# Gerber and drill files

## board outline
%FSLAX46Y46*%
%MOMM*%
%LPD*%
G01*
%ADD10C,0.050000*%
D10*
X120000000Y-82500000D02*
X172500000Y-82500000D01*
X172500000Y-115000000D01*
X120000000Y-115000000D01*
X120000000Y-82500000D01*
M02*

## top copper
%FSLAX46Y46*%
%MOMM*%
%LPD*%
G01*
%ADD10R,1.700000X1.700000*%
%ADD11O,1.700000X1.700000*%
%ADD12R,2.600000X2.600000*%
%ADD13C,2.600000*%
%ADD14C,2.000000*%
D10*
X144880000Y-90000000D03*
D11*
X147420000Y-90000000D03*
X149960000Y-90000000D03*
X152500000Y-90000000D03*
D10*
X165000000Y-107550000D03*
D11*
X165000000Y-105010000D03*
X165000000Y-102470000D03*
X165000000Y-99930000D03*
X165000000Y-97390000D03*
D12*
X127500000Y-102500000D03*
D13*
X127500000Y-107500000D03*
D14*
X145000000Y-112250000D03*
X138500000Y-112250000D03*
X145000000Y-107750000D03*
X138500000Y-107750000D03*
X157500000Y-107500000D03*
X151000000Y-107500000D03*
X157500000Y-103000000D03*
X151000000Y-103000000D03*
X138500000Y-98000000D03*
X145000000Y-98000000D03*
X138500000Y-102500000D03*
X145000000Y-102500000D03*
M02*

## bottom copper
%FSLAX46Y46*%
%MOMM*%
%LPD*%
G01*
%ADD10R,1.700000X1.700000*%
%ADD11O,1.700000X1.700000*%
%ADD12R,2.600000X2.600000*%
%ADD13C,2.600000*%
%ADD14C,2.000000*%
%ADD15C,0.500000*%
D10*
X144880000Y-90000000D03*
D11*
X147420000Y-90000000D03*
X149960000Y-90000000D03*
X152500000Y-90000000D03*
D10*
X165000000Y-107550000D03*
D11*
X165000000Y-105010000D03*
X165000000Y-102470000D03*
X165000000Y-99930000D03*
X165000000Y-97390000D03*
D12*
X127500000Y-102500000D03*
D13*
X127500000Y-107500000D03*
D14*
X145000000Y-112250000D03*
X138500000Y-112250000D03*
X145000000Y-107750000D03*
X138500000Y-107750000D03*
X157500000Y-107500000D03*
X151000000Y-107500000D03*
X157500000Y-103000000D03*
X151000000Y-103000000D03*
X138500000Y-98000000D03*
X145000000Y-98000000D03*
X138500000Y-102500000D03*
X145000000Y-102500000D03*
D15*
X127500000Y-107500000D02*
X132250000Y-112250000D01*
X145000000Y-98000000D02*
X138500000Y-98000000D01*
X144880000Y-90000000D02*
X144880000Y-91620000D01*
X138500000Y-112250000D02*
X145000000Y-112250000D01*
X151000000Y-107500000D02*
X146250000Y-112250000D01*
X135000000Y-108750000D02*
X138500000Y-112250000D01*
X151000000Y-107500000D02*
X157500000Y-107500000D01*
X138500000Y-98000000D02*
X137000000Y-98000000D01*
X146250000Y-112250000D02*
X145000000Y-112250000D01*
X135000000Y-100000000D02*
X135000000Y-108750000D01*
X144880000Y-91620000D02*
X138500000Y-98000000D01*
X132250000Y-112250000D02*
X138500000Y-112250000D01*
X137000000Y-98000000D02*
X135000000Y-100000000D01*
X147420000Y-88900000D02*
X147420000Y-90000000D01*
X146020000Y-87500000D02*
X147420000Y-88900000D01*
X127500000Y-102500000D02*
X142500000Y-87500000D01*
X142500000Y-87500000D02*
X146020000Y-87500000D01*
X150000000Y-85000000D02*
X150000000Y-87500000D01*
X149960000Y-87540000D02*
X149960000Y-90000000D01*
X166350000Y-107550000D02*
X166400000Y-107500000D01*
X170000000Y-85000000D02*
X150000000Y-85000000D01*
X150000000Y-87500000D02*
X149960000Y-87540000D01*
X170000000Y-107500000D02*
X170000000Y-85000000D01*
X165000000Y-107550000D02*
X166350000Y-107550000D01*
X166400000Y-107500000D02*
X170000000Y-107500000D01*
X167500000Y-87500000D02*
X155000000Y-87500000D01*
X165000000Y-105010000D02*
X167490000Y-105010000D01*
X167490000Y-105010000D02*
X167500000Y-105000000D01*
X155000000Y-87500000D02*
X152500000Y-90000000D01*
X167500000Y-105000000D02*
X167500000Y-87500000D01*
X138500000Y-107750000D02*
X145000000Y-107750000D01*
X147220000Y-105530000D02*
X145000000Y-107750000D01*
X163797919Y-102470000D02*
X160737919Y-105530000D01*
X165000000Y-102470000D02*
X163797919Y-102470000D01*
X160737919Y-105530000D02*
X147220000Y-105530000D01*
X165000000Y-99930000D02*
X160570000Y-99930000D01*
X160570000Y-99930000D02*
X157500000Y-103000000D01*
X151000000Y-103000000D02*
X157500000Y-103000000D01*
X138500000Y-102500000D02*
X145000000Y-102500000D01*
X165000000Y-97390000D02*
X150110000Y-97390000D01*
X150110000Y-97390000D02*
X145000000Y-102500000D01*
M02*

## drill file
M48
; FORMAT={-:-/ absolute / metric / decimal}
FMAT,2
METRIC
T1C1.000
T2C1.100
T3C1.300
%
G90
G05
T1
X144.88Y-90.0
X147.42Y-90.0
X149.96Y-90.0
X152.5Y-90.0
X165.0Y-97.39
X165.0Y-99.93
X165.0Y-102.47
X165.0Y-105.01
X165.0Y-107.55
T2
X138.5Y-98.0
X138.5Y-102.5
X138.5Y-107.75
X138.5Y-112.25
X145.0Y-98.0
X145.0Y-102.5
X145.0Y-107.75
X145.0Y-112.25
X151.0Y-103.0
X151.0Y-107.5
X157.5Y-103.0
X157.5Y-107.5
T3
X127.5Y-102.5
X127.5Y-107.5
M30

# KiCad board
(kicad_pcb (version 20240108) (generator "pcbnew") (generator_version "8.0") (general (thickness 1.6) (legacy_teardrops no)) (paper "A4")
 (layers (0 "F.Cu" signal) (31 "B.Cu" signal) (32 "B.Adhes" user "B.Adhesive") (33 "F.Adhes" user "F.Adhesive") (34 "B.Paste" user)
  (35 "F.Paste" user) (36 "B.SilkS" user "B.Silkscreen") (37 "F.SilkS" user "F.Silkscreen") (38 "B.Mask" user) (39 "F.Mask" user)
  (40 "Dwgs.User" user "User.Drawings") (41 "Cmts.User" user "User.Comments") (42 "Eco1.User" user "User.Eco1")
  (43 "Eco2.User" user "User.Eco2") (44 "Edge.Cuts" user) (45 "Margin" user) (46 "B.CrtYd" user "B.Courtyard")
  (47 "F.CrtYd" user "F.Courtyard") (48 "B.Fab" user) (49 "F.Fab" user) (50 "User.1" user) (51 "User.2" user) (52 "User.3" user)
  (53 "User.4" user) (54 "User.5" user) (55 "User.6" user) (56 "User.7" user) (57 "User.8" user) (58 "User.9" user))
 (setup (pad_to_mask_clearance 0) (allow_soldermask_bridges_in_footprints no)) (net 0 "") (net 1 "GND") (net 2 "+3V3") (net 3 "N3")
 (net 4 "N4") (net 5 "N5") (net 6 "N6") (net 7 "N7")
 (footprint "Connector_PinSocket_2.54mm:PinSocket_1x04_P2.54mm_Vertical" (layer "F.Cu") (at 144.88 90 90)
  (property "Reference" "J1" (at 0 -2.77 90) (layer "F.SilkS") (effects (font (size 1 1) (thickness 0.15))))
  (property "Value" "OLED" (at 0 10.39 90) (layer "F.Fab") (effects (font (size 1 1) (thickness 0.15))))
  (pad "1" thru_hole rect (at 0 0 90) (size 1.7 1.7) (drill 1) (layers "*.Cu" "*.Mask") (remove_unused_layers no) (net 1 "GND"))
  (pad "2" thru_hole oval (at 0 2.54 90) (size 1.7 1.7) (drill 1) (layers "*.Cu" "*.Mask") (remove_unused_layers no) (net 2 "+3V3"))
  (pad "3" thru_hole oval (at 0 5.08 90) (size 1.7 1.7) (drill 1) (layers "*.Cu" "*.Mask") (remove_unused_layers no) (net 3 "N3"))
  (pad "4" thru_hole oval (at 0 7.62 90) (size 1.7 1.7) (drill 1) (layers "*.Cu" "*.Mask") (remove_unused_layers no) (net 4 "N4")))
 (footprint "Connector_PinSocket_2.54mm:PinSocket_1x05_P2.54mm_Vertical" (layer "F.Cu") (at 165 107.55 180)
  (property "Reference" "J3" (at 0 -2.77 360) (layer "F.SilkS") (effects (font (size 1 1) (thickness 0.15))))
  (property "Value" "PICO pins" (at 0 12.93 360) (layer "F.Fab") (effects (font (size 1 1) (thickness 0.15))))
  (pad "1" thru_hole rect (at 0 0 180) (size 1.7 1.7) (drill 1) (layers "*.Cu" "*.Mask") (remove_unused_layers no) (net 3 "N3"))
  (pad "2" thru_hole oval (at 0 2.54 180) (size 1.7 1.7) (drill 1) (layers "*.Cu" "*.Mask") (remove_unused_layers no) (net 4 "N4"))
  (pad "3" thru_hole oval (at 0 5.08 180) (size 1.7 1.7) (drill 1) (layers "*.Cu" "*.Mask") (remove_unused_layers no) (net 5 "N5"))
  (pad "4" thru_hole oval (at 0 7.62 180) (size 1.7 1.7) (drill 1) (layers "*.Cu" "*.Mask") (remove_unused_layers no) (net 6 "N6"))
  (pad "5" thru_hole oval (at 0 10.16 180) (size 1.7 1.7) (drill 1) (layers "*.Cu" "*.Mask") (remove_unused_layers no) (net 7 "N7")))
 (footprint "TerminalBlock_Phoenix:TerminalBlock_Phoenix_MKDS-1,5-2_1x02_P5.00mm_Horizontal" (layer "F.Cu") (at 127.5 102.5 -90)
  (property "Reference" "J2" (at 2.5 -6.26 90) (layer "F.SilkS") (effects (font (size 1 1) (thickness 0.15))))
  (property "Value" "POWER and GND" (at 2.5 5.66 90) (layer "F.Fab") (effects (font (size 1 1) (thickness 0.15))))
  (pad "1" thru_hole rect (at 0 0 270) (size 2.6 2.6) (drill 1.3) (layers "*.Cu" "*.Mask") (remove_unused_layers no) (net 2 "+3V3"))
  (pad "2" thru_hole circle (at 5 0 270) (size 2.6 2.6) (drill 1.3) (layers "*.Cu" "*.Mask") (remove_unused_layers no) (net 1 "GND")))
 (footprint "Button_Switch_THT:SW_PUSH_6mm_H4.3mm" (layer "F.Cu") (at 145 112.25 180)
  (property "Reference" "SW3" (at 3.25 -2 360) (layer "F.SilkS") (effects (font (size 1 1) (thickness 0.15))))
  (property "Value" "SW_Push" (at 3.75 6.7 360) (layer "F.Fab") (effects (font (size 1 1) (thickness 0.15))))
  (pad "1" thru_hole circle (at 0 0 270) (size 2 2) (drill 1.1) (layers "*.Cu" "*.Mask") (remove_unused_layers no) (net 1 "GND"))
  (pad "1" thru_hole circle (at 6.5 0 270) (size 2 2) (drill 1.1) (layers "*.Cu" "*.Mask") (remove_unused_layers no) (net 1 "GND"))
  (pad "2" thru_hole circle (at 0 4.5 270) (size 2 2) (drill 1.1) (layers "*.Cu" "*.Mask") (remove_unused_layers no) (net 5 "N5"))
  (pad "2" thru_hole circle (at 6.5 4.5 270) (size 2 2) (drill 1.1) (layers "*.Cu" "*.Mask") (remove_unused_layers no) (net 5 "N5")))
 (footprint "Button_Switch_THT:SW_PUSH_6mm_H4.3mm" (layer "F.Cu") (at 157.5 107.5 180)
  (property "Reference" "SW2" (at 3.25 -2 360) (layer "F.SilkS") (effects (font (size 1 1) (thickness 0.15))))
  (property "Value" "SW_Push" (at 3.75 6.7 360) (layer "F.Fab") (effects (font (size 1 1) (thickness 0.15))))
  (pad "1" thru_hole circle (at 0 0 270) (size 2 2) (drill 1.1) (layers "*.Cu" "*.Mask") (remove_unused_layers no) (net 1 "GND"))
  (pad "1" thru_hole circle (at 6.5 0 270) (size 2 2) (drill 1.1) (layers "*.Cu" "*.Mask") (remove_unused_layers no) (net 1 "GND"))
  (pad "2" thru_hole circle (at 0 4.5 270) (size 2 2) (drill 1.1) (layers "*.Cu" "*.Mask") (remove_unused_layers no) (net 6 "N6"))
  (pad "2" thru_hole circle (at 6.5 4.5 270) (size 2 2) (drill 1.1) (layers "*.Cu" "*.Mask") (remove_unused_layers no) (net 6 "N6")))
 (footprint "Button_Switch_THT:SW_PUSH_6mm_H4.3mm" (layer "F.Cu") (at 138.5 98)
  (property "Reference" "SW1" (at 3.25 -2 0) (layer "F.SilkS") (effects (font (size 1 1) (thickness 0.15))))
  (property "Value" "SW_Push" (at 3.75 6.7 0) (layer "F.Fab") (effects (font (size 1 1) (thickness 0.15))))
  (pad "1" thru_hole circle (at 0 0 90) (size 2 2) (drill 1.1) (layers "*.Cu" "*.Mask") (remove_unused_layers no) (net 1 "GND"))
  (pad "1" thru_hole circle (at 6.5 0 90) (size 2 2) (drill 1.1) (layers "*.Cu" "*.Mask") (remove_unused_layers no) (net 1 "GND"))
  (pad "2" thru_hole circle (at 0 4.5 90) (size 2 2) (drill 1.1) (layers "*.Cu" "*.Mask") (remove_unused_layers no) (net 7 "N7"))
  (pad "2" thru_hole circle (at 6.5 4.5 90) (size 2 2) (drill 1.1) (layers "*.Cu" "*.Mask") (remove_unused_layers no) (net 7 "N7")))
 (gr_rect (start 120 82.5) (end 172.5 115) (stroke (width 0.05) (type default)) (fill none) (layer "Edge.Cuts"))
 (segment (start 127.5 107.5) (end 132.25 112.25) (width 0.5) (layer "B.Cu") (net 1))
 (segment (start 145 98) (end 138.5 98) (width 0.5) (layer "B.Cu") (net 1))
 (segment (start 144.88 90) (end 144.88 91.62) (width 0.5) (layer "B.Cu") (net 1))
 (segment (start 138.5 112.25) (end 145 112.25) (width 0.5) (layer "B.Cu") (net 1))
 (segment (start 151 107.5) (end 146.25 112.25) (width 0.5) (layer "B.Cu") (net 1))
 (segment (start 135 108.75) (end 138.5 112.25) (width 0.5) (layer "B.Cu") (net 1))
 (segment (start 151 107.5) (end 157.5 107.5) (width 0.5) (layer "B.Cu") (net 1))
 (segment (start 138.5 98) (end 137 98) (width 0.5) (layer "B.Cu") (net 1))
 (segment (start 146.25 112.25) (end 145 112.25) (width 0.5) (layer "B.Cu") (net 1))
 (segment (start 135 100) (end 135 108.75) (width 0.5) (layer "B.Cu") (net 1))
 (segment (start 144.88 91.62) (end 138.5 98) (width 0.5) (layer "B.Cu") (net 1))
 (segment (start 132.25 112.25) (end 138.5 112.25) (width 0.5) (layer "B.Cu") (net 1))
 (segment (start 137 98) (end 135 100) (width 0.5) (layer "B.Cu") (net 1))
 (segment (start 147.42 88.9) (end 147.42 90) (width 0.5) (layer "B.Cu") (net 2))
 (segment (start 146.02 87.5) (end 147.42 88.9) (width 0.5) (layer "B.Cu") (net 2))
 (segment (start 127.5 102.5) (end 142.5 87.5) (width 0.5) (layer "B.Cu") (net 2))
 (segment (start 142.5 87.5) (end 146.02 87.5) (width 0.5) (layer "B.Cu") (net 2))
 (segment (start 150 85) (end 150 87.5) (width 0.5) (layer "B.Cu") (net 3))
 (segment (start 149.96 87.54) (end 149.96 90) (width 0.5) (layer "B.Cu") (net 3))
 (segment (start 166.35 107.55) (end 166.4 107.5) (width 0.5) (layer "B.Cu") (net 3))
 (segment (start 170 85) (end 150 85) (width 0.5) (layer "B.Cu") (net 3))
 (segment (start 150 87.5) (end 149.96 87.54) (width 0.5) (layer "B.Cu") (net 3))
 (segment (start 170 107.5) (end 170 85) (width 0.5) (layer "B.Cu") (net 3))
 (segment (start 165 107.55) (end 166.35 107.55) (width 0.5) (layer "B.Cu") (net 3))
 (segment (start 166.4 107.5) (end 170 107.5) (width 0.5) (layer "B.Cu") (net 3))
 (segment (start 167.5 87.5) (end 155 87.5) (width 0.5) (layer "B.Cu") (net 4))
 (segment (start 165 105.01) (end 167.49 105.01) (width 0.5) (layer "B.Cu") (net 4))
 (segment (start 167.49 105.01) (end 167.5 105) (width 0.5) (layer "B.Cu") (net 4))
 (segment (start 155 87.5) (end 152.5 90) (width 0.5) (layer "B.Cu") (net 4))
 (segment (start 167.5 105) (end 167.5 87.5) (width 0.5) (layer "B.Cu") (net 4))
 (segment (start 138.5 107.75) (end 145 107.75) (width 0.5) (layer "B.Cu") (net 5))
 (segment (start 147.22 105.53) (end 145 107.75) (width 0.5) (layer "B.Cu") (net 5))
 (segment (start 163.797919 102.47) (end 160.737919 105.53) (width 0.5) (layer "B.Cu") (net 5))
 (segment (start 165 102.47) (end 163.797919 102.47) (width 0.5) (layer "B.Cu") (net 5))
 (segment (start 160.737919 105.53) (end 147.22 105.53) (width 0.5) (layer "B.Cu") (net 5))
 (segment (start 165 99.93) (end 160.57 99.93) (width 0.5) (layer "B.Cu") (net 6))
 (segment (start 160.57 99.93) (end 157.5 103) (width 0.5) (layer "B.Cu") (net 6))
 (segment (start 151 103) (end 157.5 103) (width 0.5) (layer "B.Cu") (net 6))
 (segment (start 138.5 102.5) (end 145 102.5) (width 0.5) (layer "B.Cu") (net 7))
 (segment (start 165 97.39) (end 150.11 97.39) (width 0.5) (layer "B.Cu") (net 7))
 (segment (start 150.11 97.39) (end 145 102.5) (width 0.5) (layer "B.Cu") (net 7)))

